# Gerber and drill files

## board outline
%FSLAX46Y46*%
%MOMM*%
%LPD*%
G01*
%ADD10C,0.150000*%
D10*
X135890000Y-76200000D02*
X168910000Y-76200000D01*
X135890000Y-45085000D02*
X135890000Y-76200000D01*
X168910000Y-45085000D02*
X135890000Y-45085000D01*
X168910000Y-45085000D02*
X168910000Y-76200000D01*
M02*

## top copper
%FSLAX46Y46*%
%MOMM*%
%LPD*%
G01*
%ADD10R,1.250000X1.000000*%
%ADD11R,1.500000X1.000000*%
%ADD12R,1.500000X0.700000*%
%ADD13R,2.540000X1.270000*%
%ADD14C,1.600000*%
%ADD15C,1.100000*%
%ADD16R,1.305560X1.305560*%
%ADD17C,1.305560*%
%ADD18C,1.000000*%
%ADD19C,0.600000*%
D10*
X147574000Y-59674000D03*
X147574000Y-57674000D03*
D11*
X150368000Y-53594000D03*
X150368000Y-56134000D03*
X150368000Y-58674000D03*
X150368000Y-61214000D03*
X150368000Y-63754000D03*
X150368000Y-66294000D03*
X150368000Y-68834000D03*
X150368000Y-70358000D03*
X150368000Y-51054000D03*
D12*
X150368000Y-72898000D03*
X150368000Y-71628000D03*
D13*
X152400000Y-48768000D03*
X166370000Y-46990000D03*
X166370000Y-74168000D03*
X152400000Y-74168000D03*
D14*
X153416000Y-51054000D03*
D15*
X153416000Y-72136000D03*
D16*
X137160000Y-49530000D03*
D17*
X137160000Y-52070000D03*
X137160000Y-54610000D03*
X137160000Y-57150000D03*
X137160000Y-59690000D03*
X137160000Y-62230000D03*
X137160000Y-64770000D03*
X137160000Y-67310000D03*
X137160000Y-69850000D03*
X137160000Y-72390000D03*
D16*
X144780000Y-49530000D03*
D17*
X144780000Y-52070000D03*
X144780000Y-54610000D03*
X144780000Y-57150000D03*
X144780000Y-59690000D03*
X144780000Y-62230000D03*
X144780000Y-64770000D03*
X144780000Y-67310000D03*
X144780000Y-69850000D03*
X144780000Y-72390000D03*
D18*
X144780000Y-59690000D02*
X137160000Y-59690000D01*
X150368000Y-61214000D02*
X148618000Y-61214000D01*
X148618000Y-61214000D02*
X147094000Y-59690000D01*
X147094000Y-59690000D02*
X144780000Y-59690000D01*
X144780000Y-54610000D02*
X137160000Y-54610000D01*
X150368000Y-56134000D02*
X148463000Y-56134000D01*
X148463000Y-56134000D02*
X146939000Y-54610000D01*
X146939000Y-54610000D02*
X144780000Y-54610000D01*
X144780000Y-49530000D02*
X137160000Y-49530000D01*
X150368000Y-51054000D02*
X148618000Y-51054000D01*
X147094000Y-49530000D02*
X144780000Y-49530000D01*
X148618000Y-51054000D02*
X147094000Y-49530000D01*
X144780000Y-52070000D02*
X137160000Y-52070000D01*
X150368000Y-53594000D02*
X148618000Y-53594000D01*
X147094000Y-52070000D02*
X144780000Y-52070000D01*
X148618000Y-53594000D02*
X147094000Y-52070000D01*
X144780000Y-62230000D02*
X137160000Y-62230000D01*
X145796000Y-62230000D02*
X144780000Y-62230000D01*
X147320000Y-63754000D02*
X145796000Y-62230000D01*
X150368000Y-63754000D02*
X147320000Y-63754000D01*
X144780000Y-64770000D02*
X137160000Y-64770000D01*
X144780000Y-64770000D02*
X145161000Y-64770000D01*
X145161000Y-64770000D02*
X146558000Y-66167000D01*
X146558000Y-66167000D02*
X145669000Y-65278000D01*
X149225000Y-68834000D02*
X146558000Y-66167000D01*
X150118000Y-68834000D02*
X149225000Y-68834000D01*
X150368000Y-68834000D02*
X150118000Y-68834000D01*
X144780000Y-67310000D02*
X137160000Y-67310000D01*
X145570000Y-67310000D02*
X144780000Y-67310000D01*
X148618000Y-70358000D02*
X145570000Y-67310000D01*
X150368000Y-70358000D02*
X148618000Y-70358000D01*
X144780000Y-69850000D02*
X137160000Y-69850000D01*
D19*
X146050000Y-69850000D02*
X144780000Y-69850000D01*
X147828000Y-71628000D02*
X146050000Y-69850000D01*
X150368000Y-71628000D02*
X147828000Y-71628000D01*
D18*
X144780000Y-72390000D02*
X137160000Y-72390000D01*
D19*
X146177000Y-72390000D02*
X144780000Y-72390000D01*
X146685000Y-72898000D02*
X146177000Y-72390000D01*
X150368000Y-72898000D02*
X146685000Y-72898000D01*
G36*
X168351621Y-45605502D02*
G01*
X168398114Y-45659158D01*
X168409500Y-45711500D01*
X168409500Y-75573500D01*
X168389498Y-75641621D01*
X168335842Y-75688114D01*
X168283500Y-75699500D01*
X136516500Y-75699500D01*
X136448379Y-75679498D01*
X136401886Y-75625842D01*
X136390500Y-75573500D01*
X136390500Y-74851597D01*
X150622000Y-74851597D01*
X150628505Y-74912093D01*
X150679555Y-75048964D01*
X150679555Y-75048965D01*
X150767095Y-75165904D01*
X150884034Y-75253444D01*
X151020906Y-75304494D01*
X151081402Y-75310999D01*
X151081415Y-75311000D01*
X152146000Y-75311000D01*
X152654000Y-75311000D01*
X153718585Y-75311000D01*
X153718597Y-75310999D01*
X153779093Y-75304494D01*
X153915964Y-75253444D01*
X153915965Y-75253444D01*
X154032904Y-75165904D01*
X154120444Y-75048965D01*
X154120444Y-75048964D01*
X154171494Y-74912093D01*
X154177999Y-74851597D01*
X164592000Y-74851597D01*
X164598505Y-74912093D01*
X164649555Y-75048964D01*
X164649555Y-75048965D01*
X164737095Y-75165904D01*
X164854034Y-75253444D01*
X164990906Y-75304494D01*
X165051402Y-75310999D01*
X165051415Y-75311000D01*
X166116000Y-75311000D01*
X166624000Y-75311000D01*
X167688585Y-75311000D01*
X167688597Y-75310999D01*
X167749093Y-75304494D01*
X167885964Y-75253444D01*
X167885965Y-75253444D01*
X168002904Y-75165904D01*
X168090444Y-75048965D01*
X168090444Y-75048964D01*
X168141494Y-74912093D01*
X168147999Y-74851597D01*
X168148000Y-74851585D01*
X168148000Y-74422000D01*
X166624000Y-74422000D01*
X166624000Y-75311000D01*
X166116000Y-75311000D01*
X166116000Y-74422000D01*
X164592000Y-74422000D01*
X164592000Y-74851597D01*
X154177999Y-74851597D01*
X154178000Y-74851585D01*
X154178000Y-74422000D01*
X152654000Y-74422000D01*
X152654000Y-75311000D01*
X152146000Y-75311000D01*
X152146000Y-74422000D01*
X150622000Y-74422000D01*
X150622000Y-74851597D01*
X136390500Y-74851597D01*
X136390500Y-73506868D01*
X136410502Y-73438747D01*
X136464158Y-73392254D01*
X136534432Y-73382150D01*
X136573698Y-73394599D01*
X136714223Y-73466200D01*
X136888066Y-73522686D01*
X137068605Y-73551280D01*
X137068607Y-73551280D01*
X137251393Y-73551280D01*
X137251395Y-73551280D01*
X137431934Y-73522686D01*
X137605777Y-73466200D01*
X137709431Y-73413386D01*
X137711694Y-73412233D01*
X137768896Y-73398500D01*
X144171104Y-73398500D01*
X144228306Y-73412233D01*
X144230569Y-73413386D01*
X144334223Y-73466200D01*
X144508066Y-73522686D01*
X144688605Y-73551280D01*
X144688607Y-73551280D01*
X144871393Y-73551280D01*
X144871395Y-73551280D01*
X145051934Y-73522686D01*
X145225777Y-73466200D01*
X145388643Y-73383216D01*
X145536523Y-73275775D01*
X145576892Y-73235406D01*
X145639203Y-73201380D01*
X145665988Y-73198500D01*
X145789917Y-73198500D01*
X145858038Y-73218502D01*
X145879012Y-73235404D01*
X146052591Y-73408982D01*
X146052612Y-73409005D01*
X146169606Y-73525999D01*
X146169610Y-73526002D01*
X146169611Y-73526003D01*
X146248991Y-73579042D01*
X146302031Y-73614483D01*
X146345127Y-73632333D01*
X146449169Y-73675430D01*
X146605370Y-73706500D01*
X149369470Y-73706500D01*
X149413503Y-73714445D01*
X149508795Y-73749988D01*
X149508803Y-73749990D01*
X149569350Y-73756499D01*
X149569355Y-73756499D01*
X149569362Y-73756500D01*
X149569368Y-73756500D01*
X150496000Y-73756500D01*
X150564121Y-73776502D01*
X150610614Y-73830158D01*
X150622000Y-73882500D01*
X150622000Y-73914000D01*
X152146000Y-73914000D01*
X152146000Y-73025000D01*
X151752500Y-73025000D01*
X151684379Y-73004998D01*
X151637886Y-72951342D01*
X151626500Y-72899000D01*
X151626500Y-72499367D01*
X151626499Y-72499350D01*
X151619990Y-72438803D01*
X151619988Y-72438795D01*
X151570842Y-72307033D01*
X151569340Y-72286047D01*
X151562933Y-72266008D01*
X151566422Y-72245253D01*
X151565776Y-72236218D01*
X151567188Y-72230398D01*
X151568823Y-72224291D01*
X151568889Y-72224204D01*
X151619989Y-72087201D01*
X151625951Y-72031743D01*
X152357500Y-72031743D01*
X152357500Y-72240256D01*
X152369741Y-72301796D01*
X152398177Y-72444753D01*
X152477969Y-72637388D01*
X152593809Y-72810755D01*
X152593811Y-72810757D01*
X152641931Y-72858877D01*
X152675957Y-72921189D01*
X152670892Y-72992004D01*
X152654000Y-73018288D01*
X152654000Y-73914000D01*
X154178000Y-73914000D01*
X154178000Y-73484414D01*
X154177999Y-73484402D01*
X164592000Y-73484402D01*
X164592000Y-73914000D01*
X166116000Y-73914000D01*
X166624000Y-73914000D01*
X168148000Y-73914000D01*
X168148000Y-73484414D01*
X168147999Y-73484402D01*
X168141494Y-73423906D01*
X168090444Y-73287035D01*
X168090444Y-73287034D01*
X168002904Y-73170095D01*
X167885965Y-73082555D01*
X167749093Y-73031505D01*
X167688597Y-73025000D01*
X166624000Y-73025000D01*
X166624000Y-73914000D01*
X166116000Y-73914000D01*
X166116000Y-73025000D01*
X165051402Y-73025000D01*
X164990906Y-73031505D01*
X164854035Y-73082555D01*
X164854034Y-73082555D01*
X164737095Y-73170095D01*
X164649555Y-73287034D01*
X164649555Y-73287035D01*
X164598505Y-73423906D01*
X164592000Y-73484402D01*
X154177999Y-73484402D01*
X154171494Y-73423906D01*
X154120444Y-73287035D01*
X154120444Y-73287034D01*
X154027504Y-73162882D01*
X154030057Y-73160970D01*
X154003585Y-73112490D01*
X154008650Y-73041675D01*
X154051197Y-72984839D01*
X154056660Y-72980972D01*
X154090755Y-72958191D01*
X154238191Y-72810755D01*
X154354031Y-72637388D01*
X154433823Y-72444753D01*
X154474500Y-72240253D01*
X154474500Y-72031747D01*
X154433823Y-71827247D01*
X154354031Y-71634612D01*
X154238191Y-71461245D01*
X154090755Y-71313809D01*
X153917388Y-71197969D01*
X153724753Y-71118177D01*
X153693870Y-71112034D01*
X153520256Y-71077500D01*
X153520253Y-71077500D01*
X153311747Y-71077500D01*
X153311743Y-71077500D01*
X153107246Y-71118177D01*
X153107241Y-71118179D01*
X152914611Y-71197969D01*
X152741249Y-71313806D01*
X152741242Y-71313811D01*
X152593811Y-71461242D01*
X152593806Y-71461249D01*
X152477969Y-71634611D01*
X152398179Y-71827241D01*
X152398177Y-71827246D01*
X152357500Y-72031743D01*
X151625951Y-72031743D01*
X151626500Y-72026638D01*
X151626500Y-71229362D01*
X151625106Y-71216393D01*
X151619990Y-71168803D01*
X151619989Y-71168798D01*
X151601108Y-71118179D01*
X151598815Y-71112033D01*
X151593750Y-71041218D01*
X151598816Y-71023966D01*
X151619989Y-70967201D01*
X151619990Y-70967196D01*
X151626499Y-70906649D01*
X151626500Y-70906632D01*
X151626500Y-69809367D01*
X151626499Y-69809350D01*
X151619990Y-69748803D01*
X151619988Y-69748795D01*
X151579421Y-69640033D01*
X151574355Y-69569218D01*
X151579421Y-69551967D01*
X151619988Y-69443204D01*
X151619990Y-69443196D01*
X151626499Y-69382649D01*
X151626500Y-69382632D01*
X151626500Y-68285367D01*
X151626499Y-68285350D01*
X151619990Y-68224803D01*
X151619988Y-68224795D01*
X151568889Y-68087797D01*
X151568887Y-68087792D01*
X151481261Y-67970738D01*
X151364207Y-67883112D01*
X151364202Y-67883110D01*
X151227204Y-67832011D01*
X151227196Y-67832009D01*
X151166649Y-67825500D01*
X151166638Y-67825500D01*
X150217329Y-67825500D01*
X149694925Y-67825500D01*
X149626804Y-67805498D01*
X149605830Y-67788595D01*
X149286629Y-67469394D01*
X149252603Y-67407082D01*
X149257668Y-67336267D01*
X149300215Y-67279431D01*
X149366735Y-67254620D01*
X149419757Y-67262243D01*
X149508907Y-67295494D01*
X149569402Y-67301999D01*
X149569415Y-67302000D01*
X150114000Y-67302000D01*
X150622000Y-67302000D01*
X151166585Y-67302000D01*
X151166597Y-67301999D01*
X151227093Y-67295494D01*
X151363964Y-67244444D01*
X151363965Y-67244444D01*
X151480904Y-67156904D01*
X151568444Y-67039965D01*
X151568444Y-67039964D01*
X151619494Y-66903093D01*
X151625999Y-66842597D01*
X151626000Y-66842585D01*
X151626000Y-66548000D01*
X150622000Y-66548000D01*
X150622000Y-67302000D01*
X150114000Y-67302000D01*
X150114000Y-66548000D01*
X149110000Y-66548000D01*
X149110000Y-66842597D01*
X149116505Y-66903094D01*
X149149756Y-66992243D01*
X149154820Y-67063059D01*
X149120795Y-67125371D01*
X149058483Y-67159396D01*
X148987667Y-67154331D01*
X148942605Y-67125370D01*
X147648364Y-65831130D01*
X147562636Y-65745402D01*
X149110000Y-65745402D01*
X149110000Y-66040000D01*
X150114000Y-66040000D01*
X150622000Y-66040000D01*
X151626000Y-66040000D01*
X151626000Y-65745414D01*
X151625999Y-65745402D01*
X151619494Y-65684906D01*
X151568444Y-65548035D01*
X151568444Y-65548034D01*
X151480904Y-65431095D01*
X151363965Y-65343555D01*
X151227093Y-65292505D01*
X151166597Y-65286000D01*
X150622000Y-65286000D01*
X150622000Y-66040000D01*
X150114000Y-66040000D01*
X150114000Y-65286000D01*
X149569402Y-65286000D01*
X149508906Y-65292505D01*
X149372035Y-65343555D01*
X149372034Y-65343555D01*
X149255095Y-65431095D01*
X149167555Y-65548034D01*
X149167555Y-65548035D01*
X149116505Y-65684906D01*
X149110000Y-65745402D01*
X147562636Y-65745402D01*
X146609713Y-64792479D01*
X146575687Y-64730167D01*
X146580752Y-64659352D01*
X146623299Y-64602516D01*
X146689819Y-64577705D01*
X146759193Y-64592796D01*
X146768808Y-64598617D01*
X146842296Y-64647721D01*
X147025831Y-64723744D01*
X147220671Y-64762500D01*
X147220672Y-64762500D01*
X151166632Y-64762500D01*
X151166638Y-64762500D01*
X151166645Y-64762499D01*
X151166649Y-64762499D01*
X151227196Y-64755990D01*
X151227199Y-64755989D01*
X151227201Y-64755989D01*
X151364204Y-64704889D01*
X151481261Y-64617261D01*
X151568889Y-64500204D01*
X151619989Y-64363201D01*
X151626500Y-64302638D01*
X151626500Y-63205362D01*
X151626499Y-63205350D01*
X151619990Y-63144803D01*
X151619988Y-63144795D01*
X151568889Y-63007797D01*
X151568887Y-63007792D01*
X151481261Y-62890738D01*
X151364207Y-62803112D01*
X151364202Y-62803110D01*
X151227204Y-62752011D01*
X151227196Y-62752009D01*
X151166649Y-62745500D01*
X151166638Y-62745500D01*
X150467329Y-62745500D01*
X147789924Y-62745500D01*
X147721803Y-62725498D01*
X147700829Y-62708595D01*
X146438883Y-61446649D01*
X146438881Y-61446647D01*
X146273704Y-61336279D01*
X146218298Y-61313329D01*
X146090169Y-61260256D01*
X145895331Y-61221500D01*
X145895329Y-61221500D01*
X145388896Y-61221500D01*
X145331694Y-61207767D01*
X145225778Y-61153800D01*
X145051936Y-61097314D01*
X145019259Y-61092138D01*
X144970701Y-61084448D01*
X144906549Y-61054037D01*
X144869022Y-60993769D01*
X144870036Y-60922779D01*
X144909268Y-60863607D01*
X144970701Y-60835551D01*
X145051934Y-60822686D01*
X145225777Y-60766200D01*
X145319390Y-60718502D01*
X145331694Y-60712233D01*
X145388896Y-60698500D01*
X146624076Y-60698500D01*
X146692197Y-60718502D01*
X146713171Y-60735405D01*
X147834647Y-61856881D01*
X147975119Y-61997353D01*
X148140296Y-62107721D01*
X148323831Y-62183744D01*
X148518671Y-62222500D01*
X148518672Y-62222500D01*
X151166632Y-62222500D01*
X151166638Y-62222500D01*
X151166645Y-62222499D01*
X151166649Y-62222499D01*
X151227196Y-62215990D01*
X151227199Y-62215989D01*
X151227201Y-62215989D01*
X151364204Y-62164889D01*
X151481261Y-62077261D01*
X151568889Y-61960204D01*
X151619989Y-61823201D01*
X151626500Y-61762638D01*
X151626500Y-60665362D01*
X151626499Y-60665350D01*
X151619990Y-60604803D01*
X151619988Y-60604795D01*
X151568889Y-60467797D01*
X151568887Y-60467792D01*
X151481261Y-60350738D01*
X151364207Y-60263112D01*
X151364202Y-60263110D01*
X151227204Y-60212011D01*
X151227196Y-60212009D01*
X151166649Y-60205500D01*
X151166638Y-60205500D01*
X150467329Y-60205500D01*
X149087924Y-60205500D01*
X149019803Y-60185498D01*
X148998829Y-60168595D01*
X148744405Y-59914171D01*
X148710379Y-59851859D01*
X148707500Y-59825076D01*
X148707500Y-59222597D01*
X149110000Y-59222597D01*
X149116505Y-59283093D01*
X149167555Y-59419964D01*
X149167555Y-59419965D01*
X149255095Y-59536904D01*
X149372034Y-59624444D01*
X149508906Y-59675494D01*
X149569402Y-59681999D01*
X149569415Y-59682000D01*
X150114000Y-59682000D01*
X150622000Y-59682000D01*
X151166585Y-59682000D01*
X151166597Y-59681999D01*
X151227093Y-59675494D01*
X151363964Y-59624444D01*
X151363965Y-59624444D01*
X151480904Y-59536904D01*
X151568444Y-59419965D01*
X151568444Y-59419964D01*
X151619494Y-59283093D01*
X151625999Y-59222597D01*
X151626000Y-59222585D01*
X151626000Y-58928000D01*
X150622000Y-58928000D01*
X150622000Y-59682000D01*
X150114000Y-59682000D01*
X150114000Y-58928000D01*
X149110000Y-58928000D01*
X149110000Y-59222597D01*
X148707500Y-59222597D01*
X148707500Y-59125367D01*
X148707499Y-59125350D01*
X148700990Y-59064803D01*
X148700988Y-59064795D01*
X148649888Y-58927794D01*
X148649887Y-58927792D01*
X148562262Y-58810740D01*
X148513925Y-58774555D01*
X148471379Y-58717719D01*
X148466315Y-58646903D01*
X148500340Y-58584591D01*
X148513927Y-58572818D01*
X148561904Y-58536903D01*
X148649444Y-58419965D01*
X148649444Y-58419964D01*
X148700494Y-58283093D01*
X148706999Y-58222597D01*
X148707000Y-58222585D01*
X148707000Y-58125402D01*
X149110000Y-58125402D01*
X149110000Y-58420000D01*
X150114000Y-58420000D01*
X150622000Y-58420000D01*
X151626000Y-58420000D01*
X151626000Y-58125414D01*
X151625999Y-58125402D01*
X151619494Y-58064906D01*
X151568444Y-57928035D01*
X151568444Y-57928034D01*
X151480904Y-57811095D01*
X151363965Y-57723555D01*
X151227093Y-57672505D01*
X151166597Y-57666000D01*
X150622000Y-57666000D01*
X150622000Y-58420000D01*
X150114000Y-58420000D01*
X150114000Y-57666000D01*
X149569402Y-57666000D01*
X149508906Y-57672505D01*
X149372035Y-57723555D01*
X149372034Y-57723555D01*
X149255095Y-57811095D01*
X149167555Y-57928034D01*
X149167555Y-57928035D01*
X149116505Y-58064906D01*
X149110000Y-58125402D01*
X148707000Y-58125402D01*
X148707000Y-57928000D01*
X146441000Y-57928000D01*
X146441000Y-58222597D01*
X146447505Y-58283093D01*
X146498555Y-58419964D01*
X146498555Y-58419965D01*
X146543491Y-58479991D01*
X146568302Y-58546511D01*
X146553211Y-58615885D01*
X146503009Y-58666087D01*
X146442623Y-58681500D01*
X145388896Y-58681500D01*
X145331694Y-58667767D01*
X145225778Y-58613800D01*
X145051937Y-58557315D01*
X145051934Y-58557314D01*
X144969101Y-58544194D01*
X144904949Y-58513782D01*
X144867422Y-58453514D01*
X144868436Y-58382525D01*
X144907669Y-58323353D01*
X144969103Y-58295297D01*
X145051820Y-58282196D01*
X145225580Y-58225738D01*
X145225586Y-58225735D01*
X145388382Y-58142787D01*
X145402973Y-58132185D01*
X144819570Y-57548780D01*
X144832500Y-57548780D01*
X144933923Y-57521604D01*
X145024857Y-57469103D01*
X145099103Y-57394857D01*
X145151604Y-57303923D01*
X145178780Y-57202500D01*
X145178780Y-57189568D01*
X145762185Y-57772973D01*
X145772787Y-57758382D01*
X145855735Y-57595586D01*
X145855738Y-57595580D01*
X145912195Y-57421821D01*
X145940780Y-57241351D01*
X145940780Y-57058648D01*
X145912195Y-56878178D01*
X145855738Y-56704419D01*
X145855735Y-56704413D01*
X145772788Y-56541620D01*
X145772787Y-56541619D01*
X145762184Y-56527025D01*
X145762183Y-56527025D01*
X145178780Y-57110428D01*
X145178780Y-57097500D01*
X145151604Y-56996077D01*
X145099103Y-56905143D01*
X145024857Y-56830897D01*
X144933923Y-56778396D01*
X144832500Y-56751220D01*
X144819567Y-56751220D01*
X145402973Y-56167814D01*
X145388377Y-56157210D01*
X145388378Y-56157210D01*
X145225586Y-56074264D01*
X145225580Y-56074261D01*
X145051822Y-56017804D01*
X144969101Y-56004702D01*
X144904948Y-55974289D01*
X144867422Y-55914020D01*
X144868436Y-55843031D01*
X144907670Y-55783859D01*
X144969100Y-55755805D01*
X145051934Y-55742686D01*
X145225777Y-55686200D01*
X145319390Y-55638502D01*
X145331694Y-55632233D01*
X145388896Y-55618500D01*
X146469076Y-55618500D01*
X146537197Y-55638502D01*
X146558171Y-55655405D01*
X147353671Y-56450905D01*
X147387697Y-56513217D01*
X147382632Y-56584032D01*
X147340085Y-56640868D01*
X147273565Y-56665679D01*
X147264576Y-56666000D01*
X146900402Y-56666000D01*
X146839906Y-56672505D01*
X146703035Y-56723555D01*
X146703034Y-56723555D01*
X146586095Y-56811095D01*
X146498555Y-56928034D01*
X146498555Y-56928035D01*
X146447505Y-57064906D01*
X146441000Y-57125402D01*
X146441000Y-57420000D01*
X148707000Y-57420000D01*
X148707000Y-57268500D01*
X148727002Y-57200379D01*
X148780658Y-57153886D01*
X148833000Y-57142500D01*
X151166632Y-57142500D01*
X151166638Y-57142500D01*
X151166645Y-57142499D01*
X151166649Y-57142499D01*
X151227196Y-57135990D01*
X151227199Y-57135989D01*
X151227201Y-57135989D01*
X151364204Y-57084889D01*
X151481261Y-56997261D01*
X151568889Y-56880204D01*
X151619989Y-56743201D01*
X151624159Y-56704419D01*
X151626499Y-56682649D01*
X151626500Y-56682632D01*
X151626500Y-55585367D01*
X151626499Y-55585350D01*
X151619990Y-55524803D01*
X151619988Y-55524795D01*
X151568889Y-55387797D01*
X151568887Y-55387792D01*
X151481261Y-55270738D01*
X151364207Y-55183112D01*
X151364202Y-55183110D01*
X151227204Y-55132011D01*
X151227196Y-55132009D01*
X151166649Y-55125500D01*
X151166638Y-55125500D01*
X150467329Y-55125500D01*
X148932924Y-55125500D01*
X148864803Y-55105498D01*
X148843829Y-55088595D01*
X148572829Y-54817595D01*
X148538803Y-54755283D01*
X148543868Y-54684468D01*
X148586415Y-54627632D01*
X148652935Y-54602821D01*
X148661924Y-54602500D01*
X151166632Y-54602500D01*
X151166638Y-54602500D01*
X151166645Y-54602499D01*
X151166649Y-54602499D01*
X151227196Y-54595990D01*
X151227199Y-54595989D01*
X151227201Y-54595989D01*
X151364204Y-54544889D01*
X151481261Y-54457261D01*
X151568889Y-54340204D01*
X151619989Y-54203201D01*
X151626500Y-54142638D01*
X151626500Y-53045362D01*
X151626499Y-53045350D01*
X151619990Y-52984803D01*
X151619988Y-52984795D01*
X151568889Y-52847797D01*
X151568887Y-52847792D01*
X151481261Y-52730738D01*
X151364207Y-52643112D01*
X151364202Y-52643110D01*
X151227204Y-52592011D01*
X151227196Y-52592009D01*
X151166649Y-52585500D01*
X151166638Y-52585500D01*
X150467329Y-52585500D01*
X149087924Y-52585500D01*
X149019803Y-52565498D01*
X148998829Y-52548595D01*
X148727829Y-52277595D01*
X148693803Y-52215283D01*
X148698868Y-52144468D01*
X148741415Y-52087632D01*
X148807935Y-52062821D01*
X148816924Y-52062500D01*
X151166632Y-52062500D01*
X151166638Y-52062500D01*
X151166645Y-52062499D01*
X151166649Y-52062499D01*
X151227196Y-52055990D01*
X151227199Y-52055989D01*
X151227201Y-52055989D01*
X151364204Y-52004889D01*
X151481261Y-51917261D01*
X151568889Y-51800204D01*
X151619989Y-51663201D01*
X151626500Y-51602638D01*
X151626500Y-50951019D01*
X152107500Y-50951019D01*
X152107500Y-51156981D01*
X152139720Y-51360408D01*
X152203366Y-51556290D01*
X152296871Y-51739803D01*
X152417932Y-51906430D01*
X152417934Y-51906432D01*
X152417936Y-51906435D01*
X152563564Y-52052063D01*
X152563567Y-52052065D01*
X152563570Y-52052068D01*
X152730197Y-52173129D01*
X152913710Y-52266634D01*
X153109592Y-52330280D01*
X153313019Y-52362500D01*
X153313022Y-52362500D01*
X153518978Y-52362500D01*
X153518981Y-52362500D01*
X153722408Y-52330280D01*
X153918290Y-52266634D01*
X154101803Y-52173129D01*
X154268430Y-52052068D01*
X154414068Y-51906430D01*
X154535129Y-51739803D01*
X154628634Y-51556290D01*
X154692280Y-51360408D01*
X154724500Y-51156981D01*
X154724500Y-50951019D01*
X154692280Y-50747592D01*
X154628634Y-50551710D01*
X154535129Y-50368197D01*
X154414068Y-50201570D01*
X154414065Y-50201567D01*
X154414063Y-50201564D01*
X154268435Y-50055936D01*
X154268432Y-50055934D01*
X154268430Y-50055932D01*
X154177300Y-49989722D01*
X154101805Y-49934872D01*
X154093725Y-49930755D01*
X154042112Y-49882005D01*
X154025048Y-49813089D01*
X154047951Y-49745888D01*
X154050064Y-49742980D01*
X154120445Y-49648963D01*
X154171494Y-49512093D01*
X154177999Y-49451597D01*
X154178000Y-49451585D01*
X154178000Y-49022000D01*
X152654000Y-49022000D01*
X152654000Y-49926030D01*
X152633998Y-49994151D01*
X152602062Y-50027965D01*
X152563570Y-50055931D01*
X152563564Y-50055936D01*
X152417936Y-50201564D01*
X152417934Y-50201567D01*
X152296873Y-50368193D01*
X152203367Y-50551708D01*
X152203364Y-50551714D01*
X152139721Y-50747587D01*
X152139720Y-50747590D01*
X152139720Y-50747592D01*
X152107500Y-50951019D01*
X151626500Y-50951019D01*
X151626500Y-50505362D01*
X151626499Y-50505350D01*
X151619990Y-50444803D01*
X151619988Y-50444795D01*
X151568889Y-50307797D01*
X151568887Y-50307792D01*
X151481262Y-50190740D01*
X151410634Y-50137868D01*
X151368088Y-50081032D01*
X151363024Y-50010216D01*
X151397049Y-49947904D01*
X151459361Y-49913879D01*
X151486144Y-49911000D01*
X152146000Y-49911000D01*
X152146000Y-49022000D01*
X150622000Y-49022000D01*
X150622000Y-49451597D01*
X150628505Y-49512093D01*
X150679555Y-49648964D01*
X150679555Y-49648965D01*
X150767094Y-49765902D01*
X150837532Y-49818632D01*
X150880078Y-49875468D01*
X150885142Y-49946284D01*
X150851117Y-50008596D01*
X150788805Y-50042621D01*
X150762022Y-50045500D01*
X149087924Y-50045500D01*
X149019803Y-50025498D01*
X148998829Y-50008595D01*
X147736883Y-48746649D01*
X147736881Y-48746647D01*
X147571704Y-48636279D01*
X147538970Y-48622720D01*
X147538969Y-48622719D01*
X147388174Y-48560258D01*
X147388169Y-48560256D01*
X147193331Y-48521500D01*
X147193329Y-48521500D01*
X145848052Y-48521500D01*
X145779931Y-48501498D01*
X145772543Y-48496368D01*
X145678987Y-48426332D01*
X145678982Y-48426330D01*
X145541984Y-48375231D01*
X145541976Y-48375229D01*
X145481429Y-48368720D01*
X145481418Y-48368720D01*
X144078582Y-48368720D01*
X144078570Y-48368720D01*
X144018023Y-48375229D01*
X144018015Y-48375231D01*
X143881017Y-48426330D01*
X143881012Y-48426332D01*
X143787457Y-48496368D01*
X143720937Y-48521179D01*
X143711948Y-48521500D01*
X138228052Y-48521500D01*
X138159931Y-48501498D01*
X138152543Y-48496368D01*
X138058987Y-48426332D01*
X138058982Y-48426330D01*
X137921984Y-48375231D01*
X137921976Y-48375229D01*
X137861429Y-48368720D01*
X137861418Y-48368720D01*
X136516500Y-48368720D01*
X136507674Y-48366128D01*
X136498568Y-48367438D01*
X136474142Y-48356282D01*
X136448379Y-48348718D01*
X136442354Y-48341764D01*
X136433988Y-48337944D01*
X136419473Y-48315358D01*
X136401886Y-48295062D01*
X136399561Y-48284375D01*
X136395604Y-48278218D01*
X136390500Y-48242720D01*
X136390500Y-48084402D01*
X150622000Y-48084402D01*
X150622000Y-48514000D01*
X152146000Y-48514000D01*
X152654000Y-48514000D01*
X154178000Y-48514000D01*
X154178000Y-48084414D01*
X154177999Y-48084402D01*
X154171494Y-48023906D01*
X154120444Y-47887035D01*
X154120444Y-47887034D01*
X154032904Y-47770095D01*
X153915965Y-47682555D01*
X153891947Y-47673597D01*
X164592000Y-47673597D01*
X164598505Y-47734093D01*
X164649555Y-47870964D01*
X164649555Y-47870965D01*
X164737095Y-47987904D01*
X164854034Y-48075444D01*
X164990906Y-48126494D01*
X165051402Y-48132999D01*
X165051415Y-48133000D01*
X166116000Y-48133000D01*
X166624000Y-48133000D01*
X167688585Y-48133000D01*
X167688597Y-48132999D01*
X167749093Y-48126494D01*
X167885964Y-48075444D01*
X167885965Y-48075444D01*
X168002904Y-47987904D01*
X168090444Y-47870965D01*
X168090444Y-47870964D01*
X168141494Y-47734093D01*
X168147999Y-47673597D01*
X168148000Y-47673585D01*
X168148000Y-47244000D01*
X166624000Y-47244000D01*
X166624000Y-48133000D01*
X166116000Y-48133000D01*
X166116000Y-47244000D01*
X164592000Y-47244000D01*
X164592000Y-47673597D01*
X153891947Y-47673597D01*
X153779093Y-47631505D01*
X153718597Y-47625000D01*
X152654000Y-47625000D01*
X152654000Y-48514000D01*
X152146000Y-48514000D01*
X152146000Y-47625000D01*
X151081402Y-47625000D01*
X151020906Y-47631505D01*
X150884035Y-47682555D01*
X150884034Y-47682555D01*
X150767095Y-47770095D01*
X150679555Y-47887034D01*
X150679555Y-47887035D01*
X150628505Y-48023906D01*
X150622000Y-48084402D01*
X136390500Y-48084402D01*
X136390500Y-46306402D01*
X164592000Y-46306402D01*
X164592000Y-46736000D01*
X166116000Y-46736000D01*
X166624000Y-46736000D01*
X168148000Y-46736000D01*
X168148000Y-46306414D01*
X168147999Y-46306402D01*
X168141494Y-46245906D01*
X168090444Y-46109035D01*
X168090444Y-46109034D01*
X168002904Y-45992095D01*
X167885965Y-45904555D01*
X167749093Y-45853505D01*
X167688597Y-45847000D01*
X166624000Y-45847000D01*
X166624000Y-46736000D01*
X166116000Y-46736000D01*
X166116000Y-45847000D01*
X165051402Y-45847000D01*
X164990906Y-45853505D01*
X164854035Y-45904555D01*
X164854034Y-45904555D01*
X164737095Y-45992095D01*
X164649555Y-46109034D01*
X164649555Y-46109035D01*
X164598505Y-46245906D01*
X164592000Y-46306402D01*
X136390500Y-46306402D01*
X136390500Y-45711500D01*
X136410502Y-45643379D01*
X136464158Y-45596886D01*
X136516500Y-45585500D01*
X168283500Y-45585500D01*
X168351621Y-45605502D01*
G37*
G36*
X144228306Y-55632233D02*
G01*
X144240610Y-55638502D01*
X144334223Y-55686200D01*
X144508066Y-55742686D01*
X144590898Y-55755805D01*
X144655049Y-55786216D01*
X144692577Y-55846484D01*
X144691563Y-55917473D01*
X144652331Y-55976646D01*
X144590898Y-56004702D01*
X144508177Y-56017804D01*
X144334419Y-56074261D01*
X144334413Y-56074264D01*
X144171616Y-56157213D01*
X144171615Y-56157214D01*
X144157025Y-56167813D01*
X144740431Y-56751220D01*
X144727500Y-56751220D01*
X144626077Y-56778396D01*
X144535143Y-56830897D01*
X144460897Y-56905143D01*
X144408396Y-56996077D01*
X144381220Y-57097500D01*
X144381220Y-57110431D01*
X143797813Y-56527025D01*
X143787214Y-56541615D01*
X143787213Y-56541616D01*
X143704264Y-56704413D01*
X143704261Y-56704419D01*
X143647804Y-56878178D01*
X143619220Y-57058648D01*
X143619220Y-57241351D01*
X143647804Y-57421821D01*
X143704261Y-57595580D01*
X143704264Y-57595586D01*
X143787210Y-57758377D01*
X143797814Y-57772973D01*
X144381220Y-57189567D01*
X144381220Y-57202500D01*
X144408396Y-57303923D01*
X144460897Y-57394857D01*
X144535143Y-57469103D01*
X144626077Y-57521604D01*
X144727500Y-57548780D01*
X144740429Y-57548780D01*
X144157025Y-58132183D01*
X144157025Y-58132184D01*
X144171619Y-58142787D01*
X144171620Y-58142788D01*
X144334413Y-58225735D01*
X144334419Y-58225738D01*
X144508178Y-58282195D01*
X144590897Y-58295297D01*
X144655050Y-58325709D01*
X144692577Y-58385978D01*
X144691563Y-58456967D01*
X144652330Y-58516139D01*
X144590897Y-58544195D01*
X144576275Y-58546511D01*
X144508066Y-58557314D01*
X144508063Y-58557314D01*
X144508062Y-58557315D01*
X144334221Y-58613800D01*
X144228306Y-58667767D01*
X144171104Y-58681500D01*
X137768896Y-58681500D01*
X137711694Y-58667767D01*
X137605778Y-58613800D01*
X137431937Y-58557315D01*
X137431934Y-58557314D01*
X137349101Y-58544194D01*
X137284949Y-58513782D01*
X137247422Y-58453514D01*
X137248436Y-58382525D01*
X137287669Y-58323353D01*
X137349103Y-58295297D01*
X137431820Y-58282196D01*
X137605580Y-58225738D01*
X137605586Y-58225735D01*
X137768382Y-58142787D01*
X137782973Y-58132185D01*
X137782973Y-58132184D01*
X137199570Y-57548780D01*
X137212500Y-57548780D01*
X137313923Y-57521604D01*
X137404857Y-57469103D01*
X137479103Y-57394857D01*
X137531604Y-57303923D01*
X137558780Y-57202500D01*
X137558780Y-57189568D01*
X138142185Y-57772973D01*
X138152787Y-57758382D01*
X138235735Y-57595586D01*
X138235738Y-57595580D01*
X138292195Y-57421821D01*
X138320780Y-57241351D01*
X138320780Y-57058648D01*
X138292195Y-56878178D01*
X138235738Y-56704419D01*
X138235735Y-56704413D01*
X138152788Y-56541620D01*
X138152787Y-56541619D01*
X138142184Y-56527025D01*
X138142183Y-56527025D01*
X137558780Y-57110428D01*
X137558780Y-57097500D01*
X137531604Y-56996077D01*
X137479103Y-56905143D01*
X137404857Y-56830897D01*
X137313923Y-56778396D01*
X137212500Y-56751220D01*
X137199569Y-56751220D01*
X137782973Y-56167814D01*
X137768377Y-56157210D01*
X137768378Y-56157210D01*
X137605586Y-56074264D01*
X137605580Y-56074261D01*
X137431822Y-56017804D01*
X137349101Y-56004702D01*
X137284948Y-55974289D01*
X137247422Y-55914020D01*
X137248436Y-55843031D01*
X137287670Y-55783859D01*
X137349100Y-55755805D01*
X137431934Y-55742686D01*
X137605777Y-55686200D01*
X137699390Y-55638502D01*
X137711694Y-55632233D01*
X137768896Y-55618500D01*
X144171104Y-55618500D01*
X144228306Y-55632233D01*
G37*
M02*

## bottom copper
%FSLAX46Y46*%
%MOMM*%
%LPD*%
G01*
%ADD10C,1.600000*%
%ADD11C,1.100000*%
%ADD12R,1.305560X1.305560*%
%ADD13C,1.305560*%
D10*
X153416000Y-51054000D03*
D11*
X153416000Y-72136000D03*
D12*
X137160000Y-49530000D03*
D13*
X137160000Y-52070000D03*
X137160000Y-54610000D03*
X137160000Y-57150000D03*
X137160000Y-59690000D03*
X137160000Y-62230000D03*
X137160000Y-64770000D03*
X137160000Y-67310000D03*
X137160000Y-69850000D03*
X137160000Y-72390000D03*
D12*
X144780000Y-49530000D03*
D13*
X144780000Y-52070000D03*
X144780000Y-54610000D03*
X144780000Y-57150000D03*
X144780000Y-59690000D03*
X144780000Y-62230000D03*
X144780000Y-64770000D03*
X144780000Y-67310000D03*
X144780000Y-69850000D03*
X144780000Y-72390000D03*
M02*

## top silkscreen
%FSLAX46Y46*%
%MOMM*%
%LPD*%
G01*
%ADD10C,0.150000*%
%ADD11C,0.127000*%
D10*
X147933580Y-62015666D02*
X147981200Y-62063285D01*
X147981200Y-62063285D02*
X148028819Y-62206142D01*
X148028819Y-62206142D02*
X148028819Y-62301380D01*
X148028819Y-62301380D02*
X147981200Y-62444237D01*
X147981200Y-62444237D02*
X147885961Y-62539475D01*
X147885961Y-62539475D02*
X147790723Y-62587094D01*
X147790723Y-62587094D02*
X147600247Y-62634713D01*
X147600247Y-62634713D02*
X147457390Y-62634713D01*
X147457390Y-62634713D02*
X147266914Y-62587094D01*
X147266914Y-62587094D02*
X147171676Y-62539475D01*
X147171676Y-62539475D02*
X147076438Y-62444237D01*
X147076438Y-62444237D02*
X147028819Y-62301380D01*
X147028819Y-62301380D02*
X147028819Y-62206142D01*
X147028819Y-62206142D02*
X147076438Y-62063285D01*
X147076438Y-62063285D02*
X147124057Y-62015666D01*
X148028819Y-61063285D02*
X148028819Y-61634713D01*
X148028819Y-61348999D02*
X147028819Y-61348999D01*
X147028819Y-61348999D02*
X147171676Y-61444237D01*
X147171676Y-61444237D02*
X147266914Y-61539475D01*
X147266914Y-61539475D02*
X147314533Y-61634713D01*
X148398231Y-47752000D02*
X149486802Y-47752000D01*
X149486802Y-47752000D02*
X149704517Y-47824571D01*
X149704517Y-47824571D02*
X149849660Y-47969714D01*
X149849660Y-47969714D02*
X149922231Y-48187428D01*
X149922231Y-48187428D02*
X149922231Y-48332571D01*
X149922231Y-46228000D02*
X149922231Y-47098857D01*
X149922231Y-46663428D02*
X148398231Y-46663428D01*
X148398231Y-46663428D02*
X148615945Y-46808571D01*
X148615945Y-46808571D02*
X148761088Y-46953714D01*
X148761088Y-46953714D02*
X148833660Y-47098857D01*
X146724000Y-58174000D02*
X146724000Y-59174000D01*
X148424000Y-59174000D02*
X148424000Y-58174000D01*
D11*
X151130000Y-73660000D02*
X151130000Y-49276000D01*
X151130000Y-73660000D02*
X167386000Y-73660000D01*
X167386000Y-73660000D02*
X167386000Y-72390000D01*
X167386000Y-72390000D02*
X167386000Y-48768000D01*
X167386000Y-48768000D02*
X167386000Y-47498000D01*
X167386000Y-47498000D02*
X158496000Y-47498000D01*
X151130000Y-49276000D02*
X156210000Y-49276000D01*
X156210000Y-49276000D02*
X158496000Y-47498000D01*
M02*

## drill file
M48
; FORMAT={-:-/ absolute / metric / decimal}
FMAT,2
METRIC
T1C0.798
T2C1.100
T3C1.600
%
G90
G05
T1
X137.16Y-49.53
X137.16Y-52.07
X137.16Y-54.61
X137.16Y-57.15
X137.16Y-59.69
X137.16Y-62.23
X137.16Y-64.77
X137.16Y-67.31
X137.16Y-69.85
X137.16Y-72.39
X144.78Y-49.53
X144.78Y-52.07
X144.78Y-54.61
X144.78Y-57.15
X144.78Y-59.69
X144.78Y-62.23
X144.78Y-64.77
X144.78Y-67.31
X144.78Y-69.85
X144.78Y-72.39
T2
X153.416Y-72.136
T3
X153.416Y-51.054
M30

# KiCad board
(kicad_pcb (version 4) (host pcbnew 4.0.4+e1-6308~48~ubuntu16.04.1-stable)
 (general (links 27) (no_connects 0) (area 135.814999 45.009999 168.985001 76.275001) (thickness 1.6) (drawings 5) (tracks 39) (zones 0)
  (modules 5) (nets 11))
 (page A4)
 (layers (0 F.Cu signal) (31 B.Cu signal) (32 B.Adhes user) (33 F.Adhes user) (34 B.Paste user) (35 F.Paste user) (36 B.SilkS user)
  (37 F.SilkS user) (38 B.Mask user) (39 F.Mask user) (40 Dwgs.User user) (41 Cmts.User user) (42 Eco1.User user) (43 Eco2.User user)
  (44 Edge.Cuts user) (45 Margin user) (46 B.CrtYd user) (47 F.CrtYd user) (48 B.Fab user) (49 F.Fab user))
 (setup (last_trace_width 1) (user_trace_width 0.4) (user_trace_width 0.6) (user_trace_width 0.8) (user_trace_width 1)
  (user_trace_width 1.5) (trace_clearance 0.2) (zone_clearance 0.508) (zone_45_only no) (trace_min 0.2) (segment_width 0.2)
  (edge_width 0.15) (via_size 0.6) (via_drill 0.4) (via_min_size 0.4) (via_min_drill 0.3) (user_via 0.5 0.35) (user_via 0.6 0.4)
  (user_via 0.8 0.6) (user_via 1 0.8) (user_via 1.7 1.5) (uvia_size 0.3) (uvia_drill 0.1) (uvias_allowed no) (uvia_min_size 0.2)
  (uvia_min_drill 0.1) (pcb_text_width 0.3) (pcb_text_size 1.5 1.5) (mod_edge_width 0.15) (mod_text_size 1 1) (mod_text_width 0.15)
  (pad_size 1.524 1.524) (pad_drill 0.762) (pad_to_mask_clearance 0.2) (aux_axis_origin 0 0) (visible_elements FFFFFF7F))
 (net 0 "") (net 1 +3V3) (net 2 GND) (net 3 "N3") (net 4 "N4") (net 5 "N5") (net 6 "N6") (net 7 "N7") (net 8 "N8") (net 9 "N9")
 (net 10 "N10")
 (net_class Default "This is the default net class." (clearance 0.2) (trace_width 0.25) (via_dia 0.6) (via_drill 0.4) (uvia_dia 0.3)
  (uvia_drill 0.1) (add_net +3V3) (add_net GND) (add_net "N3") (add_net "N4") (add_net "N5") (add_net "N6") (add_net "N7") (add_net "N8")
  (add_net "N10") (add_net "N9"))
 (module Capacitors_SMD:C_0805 (layer F.Cu) (at 147.574 58.674 90)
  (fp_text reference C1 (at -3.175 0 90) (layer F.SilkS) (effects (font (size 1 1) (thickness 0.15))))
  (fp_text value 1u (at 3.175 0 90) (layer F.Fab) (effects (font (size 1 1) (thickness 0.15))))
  (fp_line (start 0.5 -0.85) (end -0.5 -0.85) (layer F.SilkS) (width 0.15))
  (fp_line (start -0.5 0.85) (end 0.5 0.85) (layer F.SilkS) (width 0.15))
  (pad 1 smd rect (at -1 0 90) (size 1 1.25) (layers F.Cu F.Paste F.Mask) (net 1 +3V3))
  (pad 2 smd rect (at 1 0 90) (size 1 1.25) (layers F.Cu F.Paste F.Mask) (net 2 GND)))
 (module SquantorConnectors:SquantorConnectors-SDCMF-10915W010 (layer F.Cu) (at 163.83 60.96 90)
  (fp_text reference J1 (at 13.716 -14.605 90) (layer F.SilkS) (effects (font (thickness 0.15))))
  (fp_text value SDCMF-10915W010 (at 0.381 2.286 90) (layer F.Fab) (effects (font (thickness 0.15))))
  (fp_line (start -12.7 -12.7) (end 11.684 -12.7) (layer F.SilkS) (width 0.127))
  (fp_line (start -12.7 -12.7) (end -12.7 3.556) (layer F.SilkS) (width 0.127))
  (fp_line (start -12.7 3.556) (end -11.43 3.556) (layer F.SilkS) (width 0.127))
  (fp_line (start -11.43 3.556) (end 12.192 3.556) (layer F.SilkS) (width 0.127))
  (fp_line (start 12.192 3.556) (end 13.462 3.556) (layer F.SilkS) (width 0.127))
  (fp_line (start 13.462 3.556) (end 13.462 -5.334) (layer F.SilkS) (width 0.127))
  (fp_line (start 11.684 -12.7) (end 11.684 -7.62) (layer F.SilkS) (width 0.127))
  (fp_line (start 11.684 -7.62) (end 13.462 -5.334) (layer F.SilkS) (width 0.127))
  (pad 1 smd rect (at 7.366 -13.462 180) (size 1.5 1) (layers F.Cu F.Paste F.Mask) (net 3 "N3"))
  (pad 2 smd rect (at 4.826 -13.462 180) (size 1.5 1) (layers F.Cu F.Paste F.Mask) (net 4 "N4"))
  (pad 3 smd rect (at 2.286 -13.462 180) (size 1.5 1) (layers F.Cu F.Paste F.Mask) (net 2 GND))
  (pad 4 smd rect (at -0.254 -13.462 180) (size 1.5 1) (layers F.Cu F.Paste F.Mask) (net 1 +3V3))
  (pad 5 smd rect (at -2.794 -13.462 180) (size 1.5 1) (layers F.Cu F.Paste F.Mask) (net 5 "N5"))
  (pad 6 smd rect (at -5.334 -13.462 180) (size 1.5 1) (layers F.Cu F.Paste F.Mask) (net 2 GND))
  (pad 7 smd rect (at -7.874 -13.462 180) (size 1.5 1) (layers F.Cu F.Paste F.Mask) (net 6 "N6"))
  (pad 8 smd rect (at -9.398 -13.462 180) (size 1.5 1) (layers F.Cu F.Paste F.Mask) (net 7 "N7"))
  (pad 9 smd rect (at 9.906 -13.462 180) (size 1.5 1) (layers F.Cu F.Paste F.Mask) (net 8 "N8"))
  (pad WP smd rect (at -11.938 -13.462 180) (size 1.5 0.7) (layers F.Cu F.Paste F.Mask) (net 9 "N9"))
  (pad CD smd rect (at -10.668 -13.462 180) (size 1.5 0.7) (layers F.Cu F.Paste F.Mask) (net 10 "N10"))
  (pad S4 smd rect (at 12.192 -11.43 180) (size 2.54 1.27) (layers F.Cu F.Paste F.Mask) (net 2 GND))
  (pad S3 smd rect (at 13.97 2.54 180) (size 2.54 1.27) (layers F.Cu F.Paste F.Mask) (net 2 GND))
  (pad S2 smd rect (at -13.208 2.54 180) (size 2.54 1.27) (layers F.Cu F.Paste F.Mask) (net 2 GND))
  (pad S1 smd rect (at -13.208 -11.43 180) (size 2.54 1.27) (layers F.Cu F.Paste F.Mask) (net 2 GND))
  (pad D1 thru_hole circle (at 9.906 -10.414 180) (size 1.6 1.6) (drill 1.6) (layers *.Cu *.Mask))
  (pad D2 thru_hole circle (at -11.176 -10.414 180) (size 1.1 1.1) (drill 1.1) (layers *.Cu *.Mask)))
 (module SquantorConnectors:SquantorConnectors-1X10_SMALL (layer B.Cu) (at 137.16 60.96 270)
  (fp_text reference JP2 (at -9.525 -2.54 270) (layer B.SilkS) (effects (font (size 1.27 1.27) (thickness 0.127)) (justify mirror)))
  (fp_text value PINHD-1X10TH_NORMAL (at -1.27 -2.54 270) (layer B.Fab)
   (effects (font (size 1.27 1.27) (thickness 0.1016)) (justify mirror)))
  (pad 1 thru_hole rect (at -11.43 0 270) (size 1.30556 1.30556) (drill 0.79756) (layers *.Cu *.Mask B.Paste B.SilkS) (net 8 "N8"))
  (pad 2 thru_hole circle (at -8.89 0 270) (size 1.30556 1.30556) (drill 0.79756) (layers *.Cu *.Mask B.Paste B.SilkS) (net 3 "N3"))
  (pad 3 thru_hole circle (at -6.35 0 270) (size 1.30556 1.30556) (drill 0.79756) (layers *.Cu *.Mask B.Paste B.SilkS) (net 4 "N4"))
  (pad 4 thru_hole circle (at -3.81 0 270) (size 1.30556 1.30556) (drill 0.79756) (layers *.Cu *.Mask B.Paste B.SilkS) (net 2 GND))
  (pad 5 thru_hole circle (at -1.27 0 270) (size 1.30556 1.30556) (drill 0.79756) (layers *.Cu *.Mask B.Paste B.SilkS) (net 1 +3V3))
  (pad 6 thru_hole circle (at 1.27 0 270) (size 1.30556 1.30556) (drill 0.79756) (layers *.Cu *.Mask B.Paste B.SilkS) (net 5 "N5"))
  (pad 7 thru_hole circle (at 3.81 0 270) (size 1.30556 1.30556) (drill 0.79756) (layers *.Cu *.Mask B.Paste B.SilkS) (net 6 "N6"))
  (pad 8 thru_hole circle (at 6.35 0 270) (size 1.30556 1.30556) (drill 0.79756) (layers *.Cu *.Mask B.Paste B.SilkS) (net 7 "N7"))
  (pad 9 thru_hole circle (at 8.89 0 270) (size 1.30556 1.30556) (drill 0.79756) (layers *.Cu *.Mask B.Paste B.SilkS) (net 10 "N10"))
  (pad 10 thru_hole circle (at 11.43 0 270) (size 1.30556 1.30556) (drill 0.79756) (layers *.Cu *.Mask B.Paste B.SilkS) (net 9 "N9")))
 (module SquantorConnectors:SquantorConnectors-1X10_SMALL (layer B.Cu) (at 144.78 60.96 270)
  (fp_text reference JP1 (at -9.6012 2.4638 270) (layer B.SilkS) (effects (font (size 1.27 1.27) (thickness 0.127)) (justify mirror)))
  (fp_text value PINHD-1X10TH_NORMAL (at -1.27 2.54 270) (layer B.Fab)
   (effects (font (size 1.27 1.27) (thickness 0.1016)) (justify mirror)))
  (pad 1 thru_hole rect (at -11.43 0 270) (size 1.30556 1.30556) (drill 0.79756) (layers *.Cu *.Mask B.Paste B.SilkS) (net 8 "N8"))
  (pad 2 thru_hole circle (at -8.89 0 270) (size 1.30556 1.30556) (drill 0.79756) (layers *.Cu *.Mask B.Paste B.SilkS) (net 3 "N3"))
  (pad 3 thru_hole circle (at -6.35 0 270) (size 1.30556 1.30556) (drill 0.79756) (layers *.Cu *.Mask B.Paste B.SilkS) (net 4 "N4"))
  (pad 4 thru_hole circle (at -3.81 0 270) (size 1.30556 1.30556) (drill 0.79756) (layers *.Cu *.Mask B.Paste B.SilkS) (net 2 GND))
  (pad 5 thru_hole circle (at -1.27 0 270) (size 1.30556 1.30556) (drill 0.79756) (layers *.Cu *.Mask B.Paste B.SilkS) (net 1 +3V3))
  (pad 6 thru_hole circle (at 1.27 0 270) (size 1.30556 1.30556) (drill 0.79756) (layers *.Cu *.Mask B.Paste B.SilkS) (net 5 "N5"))
  (pad 7 thru_hole circle (at 3.81 0 270) (size 1.30556 1.30556) (drill 0.79756) (layers *.Cu *.Mask B.Paste B.SilkS) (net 6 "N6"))
  (pad 8 thru_hole circle (at 6.35 0 270) (size 1.30556 1.30556) (drill 0.79756) (layers *.Cu *.Mask B.Paste B.SilkS) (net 7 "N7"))
  (pad 9 thru_hole circle (at 8.89 0 270) (size 1.30556 1.30556) (drill 0.79756) (layers *.Cu *.Mask B.Paste B.SilkS) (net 10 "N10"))
  (pad 10 thru_hole circle (at 11.43 0 270) (size 1.30556 1.30556) (drill 0.79756) (layers *.Cu *.Mask B.Paste B.SilkS) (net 9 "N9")))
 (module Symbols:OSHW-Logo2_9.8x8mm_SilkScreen (layer B.Cu) (at 161.925 61.595 270)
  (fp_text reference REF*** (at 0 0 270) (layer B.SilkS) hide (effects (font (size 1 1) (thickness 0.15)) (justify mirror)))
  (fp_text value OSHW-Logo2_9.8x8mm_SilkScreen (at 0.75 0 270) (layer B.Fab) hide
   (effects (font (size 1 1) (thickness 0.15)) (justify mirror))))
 (gr_line (start 135.89 76.2) (end 168.91 76.2) (angle 90) (layer Edge.Cuts) (width 0.15))
 (gr_line (start 135.89 45.085) (end 135.89 76.2) (angle 90) (layer Edge.Cuts) (width 0.15))
 (gr_line (start 168.91 45.085) (end 135.89 45.085) (angle 90) (layer Edge.Cuts) (width 0.15))
 (gr_line (start 168.91 45.085) (end 168.91 76.2) (angle 90) (layer Edge.Cuts) (width 0.15))
 (segment (start 144.78 59.69) (end 137.16 59.69) (width 1) (layer F.Cu) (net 1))
 (segment (start 150.368 61.214) (end 148.618 61.214) (width 1) (layer F.Cu) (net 1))
 (segment (start 148.618 61.214) (end 147.094 59.69) (width 1) (layer F.Cu) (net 1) (status 20))
 (segment (start 147.094 59.69) (end 144.78 59.69) (width 1) (layer F.Cu) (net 1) (status 10))
 (segment (start 144.78 54.61) (end 137.16 54.61) (width 1) (layer F.Cu) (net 4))
 (segment (start 150.368 56.134) (end 148.463 56.134) (width 1) (layer F.Cu) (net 4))
 (segment (start 148.463 56.134) (end 146.939 54.61) (width 1) (layer F.Cu) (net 4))
 (segment (start 146.939 54.61) (end 144.78 54.61) (width 1) (layer F.Cu) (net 4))
 (segment (start 144.78 49.53) (end 137.16 49.53) (width 1) (layer F.Cu) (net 8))
 (segment (start 150.368 51.054) (end 148.618 51.054) (width 1) (layer F.Cu) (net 8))
 (segment (start 147.094 49.53) (end 144.78 49.53) (width 1) (layer F.Cu) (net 8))
 (segment (start 148.618 51.054) (end 147.094 49.53) (width 1) (layer F.Cu) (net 8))
 (segment (start 144.78 52.07) (end 137.16 52.07) (width 1) (layer F.Cu) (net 3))
 (segment (start 150.368 53.594) (end 148.618 53.594) (width 1) (layer F.Cu) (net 3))
 (segment (start 147.094 52.07) (end 144.78 52.07) (width 1) (layer F.Cu) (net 3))
 (segment (start 148.618 53.594) (end 147.094 52.07) (width 1) (layer F.Cu) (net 3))
 (segment (start 144.78 62.23) (end 137.16 62.23) (width 1) (layer F.Cu) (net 5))
 (segment (start 145.796 62.23) (end 144.78 62.23) (width 1) (layer F.Cu) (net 5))
 (segment (start 147.32 63.754) (end 145.796 62.23) (width 1) (layer F.Cu) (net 5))
 (segment (start 150.368 63.754) (end 147.32 63.754) (width 1) (layer F.Cu) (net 5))
 (segment (start 144.78 64.77) (end 137.16 64.77) (width 1) (layer F.Cu) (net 6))
 (segment (start 144.78 64.77) (end 145.161 64.77) (width 1) (layer F.Cu) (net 6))
 (segment (start 145.161 64.77) (end 146.558 66.167) (width 1) (layer F.Cu) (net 6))
 (segment (start 146.558 66.167) (end 145.669 65.278) (width 1) (layer F.Cu) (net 6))
 (segment (start 149.225 68.834) (end 146.558 66.167) (width 1) (layer F.Cu) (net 6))
 (segment (start 150.118 68.834) (end 149.225 68.834) (width 1) (layer F.Cu) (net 6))
 (segment (start 150.368 68.834) (end 150.118 68.834) (width 1) (layer F.Cu) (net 6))
 (segment (start 144.78 67.31) (end 137.16 67.31) (width 1) (layer F.Cu) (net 7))
 (segment (start 145.57 67.31) (end 144.78 67.31) (width 1) (layer F.Cu) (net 7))
 (segment (start 148.618 70.358) (end 145.57 67.31) (width 1) (layer F.Cu) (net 7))
 (segment (start 150.368 70.358) (end 148.618 70.358) (width 1) (layer F.Cu) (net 7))
 (segment (start 144.78 69.85) (end 137.16 69.85) (width 1) (layer F.Cu) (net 10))
 (segment (start 146.05 69.85) (end 144.78 69.85) (width 0.6) (layer F.Cu) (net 10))
 (segment (start 147.828 71.628) (end 146.05 69.85) (width 0.6) (layer F.Cu) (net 10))
 (segment (start 150.368 71.628) (end 147.828 71.628) (width 0.6) (layer F.Cu) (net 10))
 (segment (start 144.78 72.39) (end 137.16 72.39) (width 1) (layer F.Cu) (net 9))
 (segment (start 146.177 72.39) (end 144.78 72.39) (width 0.6) (layer F.Cu) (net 9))
 (segment (start 146.685 72.898) (end 146.177 72.39) (width 0.6) (layer F.Cu) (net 9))
 (segment (start 150.368 72.898) (end 146.685 72.898) (width 0.6) (layer F.Cu) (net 9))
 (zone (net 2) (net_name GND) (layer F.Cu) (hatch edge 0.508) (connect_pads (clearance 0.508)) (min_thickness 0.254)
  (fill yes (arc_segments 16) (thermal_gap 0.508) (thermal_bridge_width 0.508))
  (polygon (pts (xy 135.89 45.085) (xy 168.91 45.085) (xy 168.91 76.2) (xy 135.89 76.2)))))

